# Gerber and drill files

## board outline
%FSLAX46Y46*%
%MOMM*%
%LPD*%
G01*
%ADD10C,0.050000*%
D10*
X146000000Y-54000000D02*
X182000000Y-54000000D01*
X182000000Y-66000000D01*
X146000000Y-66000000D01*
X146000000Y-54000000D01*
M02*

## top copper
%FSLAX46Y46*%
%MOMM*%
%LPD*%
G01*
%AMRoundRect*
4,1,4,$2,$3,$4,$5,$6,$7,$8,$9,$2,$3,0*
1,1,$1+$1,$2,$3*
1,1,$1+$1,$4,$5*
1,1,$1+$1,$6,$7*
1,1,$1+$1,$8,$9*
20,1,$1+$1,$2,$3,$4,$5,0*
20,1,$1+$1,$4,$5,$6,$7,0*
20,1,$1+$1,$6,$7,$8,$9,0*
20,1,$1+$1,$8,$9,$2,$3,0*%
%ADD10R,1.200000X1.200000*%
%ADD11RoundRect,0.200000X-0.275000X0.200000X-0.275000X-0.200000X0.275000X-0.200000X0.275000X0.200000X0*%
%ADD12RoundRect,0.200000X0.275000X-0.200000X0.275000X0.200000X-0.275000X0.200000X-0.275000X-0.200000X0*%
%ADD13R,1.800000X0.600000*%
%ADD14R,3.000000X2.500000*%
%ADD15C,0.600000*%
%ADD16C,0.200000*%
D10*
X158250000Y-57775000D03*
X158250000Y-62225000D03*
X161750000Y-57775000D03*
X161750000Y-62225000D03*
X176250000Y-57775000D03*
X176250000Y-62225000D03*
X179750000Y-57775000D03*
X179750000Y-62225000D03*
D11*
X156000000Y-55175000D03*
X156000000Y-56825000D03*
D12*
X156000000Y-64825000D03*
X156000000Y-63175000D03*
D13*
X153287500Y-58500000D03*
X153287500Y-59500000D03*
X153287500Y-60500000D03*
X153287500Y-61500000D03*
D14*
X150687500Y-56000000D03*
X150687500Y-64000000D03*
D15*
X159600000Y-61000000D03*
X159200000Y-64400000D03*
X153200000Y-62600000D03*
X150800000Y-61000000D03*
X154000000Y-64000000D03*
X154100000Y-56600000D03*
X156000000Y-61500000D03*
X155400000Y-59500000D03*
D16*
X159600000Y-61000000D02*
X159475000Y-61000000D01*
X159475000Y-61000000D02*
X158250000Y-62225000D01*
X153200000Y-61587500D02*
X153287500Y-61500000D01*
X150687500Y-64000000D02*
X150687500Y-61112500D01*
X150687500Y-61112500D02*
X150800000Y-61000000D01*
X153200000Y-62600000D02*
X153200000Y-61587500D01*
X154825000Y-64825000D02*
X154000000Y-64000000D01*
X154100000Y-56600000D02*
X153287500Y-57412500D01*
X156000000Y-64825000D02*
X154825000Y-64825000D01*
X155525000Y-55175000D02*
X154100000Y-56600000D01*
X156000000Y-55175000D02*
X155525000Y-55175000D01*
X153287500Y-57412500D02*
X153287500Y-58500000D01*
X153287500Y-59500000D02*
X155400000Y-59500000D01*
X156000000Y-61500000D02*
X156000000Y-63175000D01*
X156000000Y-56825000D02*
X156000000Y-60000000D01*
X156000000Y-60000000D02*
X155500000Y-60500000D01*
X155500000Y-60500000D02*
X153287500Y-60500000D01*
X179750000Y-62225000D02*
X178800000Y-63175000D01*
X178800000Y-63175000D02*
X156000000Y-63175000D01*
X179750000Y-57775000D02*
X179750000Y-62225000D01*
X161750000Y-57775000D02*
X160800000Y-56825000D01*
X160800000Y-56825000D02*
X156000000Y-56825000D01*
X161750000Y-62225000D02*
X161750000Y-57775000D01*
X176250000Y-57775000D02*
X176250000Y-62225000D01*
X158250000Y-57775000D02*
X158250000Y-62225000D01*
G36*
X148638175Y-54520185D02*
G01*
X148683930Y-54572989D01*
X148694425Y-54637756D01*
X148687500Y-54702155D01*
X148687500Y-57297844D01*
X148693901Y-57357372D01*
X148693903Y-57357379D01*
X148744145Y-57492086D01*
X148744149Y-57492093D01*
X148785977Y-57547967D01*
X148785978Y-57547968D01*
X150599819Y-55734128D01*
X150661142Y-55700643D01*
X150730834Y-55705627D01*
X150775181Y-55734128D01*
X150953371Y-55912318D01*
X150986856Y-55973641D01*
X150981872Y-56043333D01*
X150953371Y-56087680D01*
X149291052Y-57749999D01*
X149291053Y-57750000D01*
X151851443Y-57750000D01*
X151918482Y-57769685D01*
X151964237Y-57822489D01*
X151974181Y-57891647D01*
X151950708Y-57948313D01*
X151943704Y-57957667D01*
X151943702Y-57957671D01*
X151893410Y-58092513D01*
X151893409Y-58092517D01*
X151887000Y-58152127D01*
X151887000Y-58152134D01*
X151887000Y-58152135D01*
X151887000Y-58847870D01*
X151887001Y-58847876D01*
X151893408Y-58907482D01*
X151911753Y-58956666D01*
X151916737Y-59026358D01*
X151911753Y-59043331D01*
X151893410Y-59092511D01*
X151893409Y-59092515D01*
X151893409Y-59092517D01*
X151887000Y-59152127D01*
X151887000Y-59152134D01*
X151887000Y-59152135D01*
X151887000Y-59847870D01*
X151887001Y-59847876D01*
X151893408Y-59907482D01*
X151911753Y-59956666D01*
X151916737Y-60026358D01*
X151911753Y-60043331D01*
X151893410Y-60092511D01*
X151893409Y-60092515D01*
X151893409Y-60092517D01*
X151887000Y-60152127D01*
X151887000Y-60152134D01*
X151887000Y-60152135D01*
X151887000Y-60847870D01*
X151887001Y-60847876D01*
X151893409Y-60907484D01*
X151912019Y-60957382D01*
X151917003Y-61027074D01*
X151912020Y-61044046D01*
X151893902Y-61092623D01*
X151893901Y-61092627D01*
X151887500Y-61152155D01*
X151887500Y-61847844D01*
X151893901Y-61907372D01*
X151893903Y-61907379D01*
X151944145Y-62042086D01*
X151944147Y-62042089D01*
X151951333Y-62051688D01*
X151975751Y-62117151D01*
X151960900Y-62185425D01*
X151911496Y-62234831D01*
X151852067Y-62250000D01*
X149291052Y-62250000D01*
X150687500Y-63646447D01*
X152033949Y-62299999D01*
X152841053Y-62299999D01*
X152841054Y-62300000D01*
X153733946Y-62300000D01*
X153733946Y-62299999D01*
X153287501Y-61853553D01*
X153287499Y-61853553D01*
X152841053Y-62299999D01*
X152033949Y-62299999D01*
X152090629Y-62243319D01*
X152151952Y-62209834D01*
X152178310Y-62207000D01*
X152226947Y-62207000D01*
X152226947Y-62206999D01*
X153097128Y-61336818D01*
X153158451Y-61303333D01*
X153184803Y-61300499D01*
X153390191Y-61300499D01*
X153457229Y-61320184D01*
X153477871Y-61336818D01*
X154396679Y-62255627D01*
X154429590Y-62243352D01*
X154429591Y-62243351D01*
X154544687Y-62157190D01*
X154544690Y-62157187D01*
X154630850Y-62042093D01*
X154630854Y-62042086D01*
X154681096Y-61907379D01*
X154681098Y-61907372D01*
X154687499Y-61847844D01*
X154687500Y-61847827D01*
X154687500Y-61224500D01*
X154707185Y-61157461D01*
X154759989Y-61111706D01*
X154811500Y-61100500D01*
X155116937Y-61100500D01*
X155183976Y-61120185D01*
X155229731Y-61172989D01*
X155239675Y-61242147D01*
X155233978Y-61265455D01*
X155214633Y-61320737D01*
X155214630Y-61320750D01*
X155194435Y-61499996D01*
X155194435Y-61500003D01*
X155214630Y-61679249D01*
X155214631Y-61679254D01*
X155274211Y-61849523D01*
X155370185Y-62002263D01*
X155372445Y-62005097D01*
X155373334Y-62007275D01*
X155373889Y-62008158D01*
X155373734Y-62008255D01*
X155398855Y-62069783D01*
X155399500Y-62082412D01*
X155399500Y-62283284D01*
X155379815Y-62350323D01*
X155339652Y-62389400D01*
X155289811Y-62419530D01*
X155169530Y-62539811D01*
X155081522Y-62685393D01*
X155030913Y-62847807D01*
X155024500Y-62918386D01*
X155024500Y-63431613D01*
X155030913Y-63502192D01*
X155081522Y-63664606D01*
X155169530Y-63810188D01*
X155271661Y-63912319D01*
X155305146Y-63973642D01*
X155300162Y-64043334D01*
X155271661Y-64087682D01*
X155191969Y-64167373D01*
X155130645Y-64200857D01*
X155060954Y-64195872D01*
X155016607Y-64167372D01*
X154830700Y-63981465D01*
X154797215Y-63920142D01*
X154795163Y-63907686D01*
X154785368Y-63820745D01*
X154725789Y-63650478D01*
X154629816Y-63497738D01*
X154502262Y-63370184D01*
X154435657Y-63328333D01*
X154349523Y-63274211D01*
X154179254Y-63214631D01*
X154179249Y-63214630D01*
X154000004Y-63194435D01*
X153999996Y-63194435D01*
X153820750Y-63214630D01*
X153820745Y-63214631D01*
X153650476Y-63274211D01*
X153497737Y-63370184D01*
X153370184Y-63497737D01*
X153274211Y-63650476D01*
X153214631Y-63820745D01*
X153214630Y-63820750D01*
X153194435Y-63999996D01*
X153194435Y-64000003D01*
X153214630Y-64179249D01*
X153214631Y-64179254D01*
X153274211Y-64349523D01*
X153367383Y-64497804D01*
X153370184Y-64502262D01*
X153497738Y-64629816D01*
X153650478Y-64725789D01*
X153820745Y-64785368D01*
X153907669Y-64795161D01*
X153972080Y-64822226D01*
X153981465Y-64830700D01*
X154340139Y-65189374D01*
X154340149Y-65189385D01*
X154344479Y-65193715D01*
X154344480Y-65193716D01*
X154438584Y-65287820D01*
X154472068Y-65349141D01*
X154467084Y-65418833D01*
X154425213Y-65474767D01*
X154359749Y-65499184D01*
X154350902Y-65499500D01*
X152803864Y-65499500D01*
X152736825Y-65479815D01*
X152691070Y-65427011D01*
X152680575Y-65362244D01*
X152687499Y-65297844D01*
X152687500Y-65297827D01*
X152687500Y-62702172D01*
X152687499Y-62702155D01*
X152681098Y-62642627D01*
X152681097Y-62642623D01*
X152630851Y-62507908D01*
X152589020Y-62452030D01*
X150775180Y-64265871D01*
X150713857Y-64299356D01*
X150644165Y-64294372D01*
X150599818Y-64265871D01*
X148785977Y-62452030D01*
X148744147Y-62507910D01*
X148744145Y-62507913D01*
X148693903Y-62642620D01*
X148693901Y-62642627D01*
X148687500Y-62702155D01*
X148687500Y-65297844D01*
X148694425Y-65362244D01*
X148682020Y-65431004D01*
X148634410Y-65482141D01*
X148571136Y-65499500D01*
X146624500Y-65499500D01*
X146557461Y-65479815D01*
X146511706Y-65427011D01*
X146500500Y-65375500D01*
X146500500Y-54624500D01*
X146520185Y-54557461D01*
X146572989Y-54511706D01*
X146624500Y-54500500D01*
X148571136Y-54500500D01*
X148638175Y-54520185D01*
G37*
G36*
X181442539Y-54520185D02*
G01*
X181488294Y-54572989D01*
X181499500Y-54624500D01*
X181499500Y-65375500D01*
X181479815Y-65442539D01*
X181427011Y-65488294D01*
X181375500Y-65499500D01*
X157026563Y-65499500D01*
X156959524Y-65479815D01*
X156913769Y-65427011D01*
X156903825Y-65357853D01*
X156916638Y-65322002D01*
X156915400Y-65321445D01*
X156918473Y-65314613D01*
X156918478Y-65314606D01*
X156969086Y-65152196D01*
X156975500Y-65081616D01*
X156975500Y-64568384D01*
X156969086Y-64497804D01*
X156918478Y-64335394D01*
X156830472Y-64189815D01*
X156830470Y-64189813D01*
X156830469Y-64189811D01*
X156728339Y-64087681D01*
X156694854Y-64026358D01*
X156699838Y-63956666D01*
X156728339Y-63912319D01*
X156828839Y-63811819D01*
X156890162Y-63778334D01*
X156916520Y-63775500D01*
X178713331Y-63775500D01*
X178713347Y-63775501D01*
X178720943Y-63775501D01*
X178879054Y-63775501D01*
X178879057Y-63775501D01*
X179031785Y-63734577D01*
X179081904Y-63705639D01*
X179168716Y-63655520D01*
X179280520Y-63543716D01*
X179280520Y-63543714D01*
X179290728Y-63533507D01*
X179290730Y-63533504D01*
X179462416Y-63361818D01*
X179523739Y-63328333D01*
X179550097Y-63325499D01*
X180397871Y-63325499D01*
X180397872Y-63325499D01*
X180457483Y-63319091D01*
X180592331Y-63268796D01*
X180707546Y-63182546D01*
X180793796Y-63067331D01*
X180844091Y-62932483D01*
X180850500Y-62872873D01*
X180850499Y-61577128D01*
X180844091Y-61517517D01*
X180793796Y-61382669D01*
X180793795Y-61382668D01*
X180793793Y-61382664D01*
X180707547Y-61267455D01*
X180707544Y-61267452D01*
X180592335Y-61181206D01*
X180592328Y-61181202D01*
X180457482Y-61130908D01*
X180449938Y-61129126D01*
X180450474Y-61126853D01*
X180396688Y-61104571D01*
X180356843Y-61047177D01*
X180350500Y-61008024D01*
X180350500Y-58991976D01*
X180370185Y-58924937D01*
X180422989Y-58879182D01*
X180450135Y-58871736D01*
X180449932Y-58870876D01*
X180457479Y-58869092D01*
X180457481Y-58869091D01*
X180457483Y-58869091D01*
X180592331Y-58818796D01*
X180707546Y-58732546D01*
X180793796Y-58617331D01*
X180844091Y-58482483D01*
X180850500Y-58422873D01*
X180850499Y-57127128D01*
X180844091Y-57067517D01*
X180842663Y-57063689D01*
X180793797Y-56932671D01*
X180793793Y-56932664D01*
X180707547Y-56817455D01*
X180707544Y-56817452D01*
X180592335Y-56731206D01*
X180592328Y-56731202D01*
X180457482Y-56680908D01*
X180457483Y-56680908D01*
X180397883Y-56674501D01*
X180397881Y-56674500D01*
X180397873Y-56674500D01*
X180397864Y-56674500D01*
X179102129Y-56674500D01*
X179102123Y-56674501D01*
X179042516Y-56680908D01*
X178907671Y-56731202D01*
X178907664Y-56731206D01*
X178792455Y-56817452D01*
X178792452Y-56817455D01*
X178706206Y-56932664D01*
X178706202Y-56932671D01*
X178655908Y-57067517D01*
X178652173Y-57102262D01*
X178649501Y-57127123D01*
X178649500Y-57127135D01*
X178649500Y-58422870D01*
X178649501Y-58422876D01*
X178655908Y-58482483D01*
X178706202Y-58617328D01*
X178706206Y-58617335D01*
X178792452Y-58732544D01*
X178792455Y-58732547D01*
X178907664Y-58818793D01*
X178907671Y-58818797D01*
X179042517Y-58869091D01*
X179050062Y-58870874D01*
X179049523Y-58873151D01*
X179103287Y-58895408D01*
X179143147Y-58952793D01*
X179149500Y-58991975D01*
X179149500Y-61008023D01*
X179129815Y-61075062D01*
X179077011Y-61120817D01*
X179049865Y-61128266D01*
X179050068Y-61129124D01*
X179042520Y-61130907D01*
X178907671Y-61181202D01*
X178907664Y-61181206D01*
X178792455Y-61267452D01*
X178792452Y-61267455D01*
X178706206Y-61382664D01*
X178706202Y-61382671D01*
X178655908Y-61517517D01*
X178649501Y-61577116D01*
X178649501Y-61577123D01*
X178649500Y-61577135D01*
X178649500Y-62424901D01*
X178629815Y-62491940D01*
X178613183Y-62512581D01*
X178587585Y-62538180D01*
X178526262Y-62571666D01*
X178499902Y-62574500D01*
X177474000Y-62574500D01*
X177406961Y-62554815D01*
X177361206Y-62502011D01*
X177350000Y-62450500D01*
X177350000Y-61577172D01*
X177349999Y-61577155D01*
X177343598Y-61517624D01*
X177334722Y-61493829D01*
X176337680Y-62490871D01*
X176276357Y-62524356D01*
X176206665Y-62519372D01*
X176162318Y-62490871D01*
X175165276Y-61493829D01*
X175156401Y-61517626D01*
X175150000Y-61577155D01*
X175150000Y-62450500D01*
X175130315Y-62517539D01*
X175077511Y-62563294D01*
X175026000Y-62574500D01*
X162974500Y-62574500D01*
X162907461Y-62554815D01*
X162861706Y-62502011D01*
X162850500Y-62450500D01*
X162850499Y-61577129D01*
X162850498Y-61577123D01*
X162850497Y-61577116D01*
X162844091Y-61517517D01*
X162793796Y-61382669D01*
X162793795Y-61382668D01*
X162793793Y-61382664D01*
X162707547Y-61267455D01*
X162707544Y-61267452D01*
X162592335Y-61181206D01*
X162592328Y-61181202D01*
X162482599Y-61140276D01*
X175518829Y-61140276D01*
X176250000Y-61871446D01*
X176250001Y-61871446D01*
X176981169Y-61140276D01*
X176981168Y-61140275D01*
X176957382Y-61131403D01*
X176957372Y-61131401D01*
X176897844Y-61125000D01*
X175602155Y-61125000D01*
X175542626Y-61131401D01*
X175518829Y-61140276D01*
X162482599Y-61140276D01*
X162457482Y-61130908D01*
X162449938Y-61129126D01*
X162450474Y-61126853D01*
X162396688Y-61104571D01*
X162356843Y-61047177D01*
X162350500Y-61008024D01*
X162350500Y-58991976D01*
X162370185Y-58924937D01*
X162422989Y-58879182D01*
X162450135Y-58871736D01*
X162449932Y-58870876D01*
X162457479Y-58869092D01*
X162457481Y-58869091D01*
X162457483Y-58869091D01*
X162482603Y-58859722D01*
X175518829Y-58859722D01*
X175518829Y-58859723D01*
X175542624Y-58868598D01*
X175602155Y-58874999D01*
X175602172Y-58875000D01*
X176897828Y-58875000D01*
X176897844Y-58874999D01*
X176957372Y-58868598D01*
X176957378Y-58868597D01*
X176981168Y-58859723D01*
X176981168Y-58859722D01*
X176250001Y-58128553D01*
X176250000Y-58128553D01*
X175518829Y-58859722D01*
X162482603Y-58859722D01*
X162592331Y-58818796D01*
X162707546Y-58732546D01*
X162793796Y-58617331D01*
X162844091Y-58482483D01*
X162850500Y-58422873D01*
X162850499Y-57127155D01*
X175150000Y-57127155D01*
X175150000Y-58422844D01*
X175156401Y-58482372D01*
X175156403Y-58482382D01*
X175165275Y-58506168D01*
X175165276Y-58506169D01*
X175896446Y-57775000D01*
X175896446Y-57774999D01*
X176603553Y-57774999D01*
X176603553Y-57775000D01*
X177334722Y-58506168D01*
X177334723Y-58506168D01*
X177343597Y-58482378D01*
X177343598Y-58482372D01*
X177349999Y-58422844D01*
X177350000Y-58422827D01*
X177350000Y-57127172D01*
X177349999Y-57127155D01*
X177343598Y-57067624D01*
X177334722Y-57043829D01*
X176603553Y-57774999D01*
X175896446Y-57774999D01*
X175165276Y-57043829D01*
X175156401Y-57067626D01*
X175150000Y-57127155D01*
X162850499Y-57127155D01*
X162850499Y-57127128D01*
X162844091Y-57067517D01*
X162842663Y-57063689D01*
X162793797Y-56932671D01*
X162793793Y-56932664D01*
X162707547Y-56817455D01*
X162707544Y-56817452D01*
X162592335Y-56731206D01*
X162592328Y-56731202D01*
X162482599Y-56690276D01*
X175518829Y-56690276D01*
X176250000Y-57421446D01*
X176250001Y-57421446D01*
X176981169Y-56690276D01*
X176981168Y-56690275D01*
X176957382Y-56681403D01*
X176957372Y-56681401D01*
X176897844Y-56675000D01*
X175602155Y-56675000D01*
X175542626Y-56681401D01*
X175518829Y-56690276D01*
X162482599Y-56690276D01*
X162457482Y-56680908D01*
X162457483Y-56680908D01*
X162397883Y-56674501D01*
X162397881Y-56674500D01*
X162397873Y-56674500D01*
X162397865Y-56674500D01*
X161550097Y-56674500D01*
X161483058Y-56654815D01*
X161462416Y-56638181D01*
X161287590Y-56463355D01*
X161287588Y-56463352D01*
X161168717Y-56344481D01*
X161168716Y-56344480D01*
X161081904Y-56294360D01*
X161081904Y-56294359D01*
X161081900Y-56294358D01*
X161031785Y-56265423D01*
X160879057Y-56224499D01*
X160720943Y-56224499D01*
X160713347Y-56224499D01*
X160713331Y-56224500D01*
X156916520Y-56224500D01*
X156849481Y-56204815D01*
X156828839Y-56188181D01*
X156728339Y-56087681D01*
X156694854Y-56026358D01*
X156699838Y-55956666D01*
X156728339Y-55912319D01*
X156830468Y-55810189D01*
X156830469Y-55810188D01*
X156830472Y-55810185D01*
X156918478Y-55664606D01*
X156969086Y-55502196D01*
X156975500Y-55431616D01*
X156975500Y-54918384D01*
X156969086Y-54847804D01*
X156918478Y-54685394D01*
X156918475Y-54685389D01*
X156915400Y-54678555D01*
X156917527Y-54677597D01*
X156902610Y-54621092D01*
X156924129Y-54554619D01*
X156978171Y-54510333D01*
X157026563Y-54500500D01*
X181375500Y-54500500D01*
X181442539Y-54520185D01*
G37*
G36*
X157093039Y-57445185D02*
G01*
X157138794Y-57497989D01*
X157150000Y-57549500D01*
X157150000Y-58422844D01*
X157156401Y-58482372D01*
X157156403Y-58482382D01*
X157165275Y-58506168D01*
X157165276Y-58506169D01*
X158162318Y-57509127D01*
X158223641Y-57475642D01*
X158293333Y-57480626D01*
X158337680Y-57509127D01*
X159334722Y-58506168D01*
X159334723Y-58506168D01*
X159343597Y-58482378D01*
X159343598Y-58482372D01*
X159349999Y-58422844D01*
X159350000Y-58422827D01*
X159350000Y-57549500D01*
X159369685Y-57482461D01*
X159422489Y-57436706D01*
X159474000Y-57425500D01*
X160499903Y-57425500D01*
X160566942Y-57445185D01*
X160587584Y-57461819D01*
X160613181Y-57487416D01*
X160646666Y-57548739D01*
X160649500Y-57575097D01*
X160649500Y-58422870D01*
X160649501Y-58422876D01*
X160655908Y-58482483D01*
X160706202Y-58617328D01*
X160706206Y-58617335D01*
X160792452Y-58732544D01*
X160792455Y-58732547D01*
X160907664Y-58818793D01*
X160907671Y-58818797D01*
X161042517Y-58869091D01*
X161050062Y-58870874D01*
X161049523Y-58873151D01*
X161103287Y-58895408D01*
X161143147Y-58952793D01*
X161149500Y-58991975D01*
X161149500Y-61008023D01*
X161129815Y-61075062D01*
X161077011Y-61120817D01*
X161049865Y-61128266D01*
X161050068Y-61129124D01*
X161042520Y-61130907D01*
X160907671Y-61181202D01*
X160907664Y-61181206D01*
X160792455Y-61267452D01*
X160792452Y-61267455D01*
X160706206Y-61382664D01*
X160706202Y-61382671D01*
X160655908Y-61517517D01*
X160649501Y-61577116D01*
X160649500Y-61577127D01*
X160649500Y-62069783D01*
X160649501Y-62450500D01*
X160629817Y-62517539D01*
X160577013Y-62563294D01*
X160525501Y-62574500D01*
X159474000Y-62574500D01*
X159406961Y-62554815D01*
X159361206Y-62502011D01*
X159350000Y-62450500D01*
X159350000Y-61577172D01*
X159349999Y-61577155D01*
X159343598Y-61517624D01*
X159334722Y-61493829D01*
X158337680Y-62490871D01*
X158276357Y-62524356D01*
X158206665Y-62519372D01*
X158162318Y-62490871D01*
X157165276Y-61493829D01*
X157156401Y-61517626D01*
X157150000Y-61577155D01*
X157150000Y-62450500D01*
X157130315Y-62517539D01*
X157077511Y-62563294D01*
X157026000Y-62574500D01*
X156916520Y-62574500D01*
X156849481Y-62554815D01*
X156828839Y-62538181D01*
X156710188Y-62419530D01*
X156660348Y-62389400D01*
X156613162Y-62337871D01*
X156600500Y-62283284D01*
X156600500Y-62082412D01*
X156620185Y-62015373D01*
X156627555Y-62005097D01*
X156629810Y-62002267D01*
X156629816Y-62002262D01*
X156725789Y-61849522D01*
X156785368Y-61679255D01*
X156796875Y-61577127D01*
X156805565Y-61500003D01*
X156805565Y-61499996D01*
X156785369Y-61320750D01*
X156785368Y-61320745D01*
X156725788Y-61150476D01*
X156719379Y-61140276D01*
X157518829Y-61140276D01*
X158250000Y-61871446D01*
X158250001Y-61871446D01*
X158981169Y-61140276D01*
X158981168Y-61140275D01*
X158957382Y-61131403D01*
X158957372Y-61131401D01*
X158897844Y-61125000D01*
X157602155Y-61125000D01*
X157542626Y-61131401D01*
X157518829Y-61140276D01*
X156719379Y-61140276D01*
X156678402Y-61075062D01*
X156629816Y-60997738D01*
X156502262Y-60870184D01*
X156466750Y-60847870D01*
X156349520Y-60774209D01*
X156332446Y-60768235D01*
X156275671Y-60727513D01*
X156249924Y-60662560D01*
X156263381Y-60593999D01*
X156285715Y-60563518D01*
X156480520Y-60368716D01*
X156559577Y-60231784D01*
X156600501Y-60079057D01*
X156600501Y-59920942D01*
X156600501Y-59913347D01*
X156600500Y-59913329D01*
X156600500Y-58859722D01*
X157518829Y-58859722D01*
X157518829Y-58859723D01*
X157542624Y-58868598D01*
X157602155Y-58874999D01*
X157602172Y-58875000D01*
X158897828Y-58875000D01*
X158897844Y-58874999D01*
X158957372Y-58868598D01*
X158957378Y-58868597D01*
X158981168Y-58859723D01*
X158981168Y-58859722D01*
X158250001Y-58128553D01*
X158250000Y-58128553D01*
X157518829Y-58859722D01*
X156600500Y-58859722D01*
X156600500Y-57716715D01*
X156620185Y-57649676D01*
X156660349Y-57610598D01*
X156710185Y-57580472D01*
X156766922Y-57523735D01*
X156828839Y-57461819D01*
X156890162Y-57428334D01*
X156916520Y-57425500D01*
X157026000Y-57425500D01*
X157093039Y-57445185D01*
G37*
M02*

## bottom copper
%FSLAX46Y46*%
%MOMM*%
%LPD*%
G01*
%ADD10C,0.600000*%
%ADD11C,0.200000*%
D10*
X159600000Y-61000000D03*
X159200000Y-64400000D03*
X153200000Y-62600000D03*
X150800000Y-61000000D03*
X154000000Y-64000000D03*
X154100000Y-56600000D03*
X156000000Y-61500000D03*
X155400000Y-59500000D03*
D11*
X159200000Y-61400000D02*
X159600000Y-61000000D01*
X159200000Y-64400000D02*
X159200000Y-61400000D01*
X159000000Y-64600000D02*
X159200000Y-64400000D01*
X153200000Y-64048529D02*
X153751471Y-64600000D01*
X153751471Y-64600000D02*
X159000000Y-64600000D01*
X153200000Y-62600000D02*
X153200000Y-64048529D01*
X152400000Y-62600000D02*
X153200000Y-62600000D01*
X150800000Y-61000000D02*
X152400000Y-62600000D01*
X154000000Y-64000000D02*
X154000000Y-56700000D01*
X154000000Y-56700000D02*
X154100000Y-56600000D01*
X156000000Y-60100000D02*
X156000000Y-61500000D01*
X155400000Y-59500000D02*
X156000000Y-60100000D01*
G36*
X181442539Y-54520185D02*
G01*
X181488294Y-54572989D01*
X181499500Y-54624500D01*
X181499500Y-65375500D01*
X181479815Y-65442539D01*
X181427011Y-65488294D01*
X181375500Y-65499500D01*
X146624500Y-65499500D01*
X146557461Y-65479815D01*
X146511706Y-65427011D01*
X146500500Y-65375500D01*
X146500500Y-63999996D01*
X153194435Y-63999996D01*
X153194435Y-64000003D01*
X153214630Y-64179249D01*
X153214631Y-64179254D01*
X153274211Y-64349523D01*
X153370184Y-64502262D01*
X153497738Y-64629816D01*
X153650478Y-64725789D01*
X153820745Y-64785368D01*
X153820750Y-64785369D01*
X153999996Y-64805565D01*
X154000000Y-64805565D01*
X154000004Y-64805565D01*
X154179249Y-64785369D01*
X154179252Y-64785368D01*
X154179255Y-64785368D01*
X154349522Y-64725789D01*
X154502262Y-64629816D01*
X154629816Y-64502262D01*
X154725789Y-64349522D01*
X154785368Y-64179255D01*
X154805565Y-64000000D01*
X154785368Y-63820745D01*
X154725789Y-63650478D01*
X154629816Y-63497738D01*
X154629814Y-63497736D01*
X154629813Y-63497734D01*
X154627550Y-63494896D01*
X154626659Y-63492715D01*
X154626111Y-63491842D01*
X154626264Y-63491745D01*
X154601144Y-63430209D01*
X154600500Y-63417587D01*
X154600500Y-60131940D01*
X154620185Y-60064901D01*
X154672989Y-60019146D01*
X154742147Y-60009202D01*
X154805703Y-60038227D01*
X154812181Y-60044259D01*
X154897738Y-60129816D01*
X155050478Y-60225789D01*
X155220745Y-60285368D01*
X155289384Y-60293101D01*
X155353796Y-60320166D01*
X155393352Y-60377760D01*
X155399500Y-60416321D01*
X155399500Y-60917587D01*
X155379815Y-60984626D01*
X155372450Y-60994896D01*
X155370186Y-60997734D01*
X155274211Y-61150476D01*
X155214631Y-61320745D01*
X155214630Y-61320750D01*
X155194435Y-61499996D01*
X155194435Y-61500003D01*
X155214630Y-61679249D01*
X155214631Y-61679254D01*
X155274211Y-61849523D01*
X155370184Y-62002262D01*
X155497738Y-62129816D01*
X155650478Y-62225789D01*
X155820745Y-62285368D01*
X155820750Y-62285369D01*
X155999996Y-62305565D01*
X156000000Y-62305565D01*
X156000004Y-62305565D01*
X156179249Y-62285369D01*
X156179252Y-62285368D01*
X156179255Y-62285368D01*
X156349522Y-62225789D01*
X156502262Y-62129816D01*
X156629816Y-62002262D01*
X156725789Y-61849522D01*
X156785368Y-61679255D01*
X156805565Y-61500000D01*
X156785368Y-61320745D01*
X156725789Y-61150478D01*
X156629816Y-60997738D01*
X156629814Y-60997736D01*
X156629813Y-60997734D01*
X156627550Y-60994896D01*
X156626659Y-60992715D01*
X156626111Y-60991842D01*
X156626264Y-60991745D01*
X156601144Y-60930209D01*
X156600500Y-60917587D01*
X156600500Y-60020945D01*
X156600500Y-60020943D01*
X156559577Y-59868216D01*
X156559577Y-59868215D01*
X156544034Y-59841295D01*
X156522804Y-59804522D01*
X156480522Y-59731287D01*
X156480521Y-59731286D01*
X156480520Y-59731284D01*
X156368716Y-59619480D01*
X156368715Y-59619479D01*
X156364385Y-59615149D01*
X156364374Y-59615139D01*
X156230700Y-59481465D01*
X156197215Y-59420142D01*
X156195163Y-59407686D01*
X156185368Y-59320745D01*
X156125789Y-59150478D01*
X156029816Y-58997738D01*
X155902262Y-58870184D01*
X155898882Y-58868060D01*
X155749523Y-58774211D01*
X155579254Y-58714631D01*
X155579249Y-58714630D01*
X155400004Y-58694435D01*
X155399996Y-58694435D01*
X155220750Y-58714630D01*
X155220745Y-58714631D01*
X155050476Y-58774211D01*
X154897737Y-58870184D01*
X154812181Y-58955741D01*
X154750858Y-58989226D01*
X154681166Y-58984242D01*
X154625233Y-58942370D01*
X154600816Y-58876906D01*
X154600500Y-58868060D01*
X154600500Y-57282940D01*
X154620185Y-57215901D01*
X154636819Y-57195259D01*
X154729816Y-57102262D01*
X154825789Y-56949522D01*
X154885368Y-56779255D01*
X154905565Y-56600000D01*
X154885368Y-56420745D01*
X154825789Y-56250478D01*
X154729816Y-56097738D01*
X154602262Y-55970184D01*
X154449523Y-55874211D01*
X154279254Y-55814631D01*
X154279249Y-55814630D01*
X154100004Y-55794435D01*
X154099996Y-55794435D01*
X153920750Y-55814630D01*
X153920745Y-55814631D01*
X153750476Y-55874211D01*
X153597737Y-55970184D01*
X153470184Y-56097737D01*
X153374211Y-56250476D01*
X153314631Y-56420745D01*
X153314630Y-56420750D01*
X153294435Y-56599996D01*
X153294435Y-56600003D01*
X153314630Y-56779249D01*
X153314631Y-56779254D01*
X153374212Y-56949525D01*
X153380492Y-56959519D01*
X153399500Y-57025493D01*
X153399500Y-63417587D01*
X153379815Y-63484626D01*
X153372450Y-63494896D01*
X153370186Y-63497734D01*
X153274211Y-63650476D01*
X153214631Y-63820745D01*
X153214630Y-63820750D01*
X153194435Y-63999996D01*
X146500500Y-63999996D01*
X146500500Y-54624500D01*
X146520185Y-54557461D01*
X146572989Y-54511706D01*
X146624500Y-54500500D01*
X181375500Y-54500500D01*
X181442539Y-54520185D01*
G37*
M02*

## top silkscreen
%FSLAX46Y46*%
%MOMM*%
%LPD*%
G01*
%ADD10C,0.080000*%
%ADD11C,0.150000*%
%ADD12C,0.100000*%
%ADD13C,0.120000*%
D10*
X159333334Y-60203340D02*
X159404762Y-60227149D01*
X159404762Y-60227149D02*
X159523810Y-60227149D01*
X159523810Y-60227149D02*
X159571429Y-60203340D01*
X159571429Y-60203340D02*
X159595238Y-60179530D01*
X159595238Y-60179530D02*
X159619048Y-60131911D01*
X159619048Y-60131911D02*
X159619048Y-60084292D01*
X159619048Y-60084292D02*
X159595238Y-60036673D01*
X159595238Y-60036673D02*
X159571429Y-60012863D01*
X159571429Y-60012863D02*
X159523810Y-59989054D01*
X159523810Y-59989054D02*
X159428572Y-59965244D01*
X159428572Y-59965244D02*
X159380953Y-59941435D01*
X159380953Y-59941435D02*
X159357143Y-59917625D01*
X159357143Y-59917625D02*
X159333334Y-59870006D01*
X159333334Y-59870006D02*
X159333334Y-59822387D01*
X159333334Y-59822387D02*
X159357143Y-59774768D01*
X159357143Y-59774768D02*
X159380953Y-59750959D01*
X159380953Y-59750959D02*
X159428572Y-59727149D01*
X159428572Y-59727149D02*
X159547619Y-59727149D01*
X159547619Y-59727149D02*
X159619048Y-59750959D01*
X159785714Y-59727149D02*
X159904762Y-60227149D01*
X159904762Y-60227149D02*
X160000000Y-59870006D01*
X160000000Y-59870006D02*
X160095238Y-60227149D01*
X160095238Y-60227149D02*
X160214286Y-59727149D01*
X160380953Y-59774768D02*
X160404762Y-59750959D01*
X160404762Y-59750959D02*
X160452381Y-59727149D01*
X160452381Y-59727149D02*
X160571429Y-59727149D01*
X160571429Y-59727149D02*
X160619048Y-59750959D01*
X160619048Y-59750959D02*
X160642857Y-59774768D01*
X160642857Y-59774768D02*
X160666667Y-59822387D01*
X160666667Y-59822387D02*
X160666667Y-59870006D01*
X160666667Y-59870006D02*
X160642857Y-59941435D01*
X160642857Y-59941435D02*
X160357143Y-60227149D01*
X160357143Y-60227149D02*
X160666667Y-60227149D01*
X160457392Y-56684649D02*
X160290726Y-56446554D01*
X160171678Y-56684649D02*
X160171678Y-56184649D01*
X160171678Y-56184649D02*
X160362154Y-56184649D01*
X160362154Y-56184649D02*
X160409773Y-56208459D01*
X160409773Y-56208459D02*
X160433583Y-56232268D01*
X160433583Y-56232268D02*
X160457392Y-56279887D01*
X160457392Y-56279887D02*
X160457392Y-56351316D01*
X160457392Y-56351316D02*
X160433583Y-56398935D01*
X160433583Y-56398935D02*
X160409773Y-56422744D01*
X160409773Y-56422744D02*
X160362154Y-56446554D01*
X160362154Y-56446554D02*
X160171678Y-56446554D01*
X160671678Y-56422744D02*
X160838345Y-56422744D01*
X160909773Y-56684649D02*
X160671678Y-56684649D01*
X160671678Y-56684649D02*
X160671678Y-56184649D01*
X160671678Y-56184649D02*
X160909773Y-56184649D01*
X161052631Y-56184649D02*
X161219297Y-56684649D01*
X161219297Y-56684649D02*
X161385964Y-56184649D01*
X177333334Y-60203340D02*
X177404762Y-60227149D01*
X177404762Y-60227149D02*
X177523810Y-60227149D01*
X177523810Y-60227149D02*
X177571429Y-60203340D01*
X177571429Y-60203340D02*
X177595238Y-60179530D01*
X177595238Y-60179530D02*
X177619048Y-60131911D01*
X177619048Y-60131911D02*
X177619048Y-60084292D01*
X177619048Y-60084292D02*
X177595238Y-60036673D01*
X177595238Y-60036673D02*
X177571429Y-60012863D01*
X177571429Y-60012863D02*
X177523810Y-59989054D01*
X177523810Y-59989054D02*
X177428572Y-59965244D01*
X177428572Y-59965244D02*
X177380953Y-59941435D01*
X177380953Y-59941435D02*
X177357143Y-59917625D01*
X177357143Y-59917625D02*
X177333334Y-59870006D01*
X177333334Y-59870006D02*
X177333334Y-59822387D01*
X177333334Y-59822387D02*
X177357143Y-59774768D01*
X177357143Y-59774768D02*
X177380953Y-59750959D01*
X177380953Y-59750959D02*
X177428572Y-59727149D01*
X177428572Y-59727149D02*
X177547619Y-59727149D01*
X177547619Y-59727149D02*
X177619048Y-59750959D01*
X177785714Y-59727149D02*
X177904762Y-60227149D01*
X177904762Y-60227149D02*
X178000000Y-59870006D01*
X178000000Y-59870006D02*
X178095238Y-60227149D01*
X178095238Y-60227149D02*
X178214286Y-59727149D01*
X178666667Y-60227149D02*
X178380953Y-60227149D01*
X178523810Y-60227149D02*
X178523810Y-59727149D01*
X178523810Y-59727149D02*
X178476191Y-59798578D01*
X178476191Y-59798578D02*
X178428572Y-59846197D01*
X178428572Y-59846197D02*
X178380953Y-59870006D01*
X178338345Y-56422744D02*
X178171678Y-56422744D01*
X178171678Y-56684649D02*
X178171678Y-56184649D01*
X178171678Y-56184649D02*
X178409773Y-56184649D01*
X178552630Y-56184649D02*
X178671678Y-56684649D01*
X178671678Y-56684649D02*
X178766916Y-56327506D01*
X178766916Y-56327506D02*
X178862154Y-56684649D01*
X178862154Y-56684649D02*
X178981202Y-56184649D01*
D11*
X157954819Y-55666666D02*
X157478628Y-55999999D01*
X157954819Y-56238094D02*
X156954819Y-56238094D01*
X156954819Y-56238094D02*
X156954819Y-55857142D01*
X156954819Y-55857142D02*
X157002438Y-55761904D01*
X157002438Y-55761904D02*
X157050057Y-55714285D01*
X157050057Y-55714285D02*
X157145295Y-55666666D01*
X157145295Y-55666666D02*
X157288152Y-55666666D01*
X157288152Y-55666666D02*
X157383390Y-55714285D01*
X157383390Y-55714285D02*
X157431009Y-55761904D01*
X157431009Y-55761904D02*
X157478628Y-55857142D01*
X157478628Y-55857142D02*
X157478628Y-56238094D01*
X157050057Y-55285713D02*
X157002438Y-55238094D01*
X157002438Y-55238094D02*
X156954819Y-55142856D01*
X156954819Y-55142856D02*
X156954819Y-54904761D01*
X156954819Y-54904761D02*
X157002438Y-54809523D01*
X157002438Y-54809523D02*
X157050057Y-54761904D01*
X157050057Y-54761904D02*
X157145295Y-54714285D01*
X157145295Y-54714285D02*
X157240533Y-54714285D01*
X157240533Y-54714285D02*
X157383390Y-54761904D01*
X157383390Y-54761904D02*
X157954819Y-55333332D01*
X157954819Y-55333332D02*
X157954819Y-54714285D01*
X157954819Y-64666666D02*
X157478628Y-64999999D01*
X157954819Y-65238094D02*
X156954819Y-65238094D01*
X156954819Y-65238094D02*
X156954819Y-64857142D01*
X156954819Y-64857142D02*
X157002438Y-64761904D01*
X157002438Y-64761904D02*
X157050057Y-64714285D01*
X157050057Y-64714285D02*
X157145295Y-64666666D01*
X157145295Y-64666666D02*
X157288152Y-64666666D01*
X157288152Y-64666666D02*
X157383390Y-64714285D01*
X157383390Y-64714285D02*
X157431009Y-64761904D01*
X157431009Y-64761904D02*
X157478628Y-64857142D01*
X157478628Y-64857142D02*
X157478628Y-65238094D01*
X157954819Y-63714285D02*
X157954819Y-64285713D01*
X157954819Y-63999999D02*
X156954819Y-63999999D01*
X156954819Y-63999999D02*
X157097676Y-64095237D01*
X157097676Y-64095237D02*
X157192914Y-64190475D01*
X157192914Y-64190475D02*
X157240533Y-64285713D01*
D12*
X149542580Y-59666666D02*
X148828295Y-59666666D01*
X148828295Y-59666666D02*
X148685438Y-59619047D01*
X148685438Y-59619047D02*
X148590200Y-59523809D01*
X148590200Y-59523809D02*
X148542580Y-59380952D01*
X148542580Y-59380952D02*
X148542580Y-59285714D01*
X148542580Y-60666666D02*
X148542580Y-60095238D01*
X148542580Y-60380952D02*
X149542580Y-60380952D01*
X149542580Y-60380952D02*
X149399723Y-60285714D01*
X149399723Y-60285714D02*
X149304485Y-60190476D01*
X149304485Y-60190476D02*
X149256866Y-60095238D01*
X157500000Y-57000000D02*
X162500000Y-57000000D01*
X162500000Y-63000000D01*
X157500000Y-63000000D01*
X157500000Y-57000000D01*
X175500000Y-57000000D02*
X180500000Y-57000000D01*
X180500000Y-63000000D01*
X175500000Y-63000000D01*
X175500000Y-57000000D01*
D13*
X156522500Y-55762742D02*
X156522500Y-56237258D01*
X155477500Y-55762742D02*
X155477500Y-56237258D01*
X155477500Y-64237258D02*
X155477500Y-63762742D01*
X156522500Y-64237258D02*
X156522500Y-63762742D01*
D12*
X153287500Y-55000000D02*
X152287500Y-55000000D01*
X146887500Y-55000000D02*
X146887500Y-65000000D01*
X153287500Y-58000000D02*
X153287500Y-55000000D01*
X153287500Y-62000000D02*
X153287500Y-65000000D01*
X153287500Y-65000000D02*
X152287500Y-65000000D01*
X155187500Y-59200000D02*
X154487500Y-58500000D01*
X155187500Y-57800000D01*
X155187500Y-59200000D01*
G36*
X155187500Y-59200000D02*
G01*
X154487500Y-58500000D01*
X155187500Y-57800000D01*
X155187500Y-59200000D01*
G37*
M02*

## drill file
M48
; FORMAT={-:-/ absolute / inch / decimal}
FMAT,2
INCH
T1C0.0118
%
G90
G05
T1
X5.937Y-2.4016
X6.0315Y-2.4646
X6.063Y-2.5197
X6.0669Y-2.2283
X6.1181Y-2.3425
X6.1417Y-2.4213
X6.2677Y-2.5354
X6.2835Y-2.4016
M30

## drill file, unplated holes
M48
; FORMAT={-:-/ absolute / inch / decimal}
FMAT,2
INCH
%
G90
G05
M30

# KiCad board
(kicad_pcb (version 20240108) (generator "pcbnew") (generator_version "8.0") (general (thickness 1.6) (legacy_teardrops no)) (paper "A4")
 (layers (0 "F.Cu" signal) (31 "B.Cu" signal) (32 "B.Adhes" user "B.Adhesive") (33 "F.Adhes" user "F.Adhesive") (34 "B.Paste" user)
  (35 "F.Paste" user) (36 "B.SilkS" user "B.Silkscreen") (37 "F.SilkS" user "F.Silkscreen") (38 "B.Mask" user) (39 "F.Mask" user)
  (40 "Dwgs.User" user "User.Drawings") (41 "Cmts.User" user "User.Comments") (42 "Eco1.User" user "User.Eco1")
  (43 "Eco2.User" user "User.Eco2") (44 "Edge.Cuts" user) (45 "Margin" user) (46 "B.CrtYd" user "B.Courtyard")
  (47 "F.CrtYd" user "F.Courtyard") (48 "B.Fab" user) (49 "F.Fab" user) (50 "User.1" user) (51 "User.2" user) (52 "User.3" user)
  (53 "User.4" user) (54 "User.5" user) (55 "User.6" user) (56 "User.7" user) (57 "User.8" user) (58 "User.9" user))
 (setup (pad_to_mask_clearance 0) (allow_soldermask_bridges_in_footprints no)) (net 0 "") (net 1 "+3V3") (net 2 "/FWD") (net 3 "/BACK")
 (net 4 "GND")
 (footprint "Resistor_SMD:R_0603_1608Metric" (layer "F.Cu") (at 156 64 90)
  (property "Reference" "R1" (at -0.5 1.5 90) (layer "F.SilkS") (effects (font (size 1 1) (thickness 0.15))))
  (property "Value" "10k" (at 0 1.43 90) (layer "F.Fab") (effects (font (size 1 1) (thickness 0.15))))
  (fp_line (start -0.237258 -0.5225) (end 0.237258 -0.5225) (stroke (width 0.12) (type solid)) (layer "F.SilkS"))
  (fp_line (start -0.237258 0.5225) (end 0.237258 0.5225) (stroke (width 0.12) (type solid)) (layer "F.SilkS"))
  (pad "1" smd roundrect (at -0.825 0 90) (size 0.8 0.95) (layers "F.Cu" "F.Paste" "F.Mask") (roundrect_rratio 0.25) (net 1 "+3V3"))
  (pad "2" smd roundrect (at 0.825 0 90) (size 0.8 0.95) (layers "F.Cu" "F.Paste" "F.Mask") (roundrect_rratio 0.25) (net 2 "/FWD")))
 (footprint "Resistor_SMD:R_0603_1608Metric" (layer "F.Cu") (at 156 56 -90)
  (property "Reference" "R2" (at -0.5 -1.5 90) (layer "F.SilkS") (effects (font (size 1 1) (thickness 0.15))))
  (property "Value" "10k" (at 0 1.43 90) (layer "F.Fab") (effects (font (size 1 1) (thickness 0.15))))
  (fp_line (start -0.237258 0.5225) (end 0.237258 0.5225) (stroke (width 0.12) (type solid)) (layer "F.SilkS"))
  (fp_line (start -0.237258 -0.5225) (end 0.237258 -0.5225) (stroke (width 0.12) (type solid)) (layer "F.SilkS"))
  (pad "1" smd roundrect (at -0.825 0 270) (size 0.8 0.95) (layers "F.Cu" "F.Paste" "F.Mask") (roundrect_rratio 0.25) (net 1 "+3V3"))
  (pad "2" smd roundrect (at 0.825 0 270) (size 0.8 0.95) (layers "F.Cu" "F.Paste" "F.Mask") (roundrect_rratio 0.25) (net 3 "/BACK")))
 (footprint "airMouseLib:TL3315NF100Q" (layer "F.Cu") (at 178 60)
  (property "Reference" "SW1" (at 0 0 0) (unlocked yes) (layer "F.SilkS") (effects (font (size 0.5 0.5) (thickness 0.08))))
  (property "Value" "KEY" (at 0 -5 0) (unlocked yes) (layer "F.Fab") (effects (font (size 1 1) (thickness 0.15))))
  (fp_rect (start -2.5 -3) (end 2.5 3) (stroke (width 0.1) (type default)) (fill none) (layer "F.SilkS"))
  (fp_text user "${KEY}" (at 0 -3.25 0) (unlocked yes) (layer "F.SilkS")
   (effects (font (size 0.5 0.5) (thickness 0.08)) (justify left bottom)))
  (pad "1" smd rect (at -1.75 -2.225) (size 1.2 1.2) (layers "F.Cu" "F.Paste" "F.Mask") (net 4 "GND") (thermal_bridge_angle 45))
  (pad "1" smd rect (at -1.75 2.225 180) (size 1.2 1.2) (layers "F.Cu" "F.Paste" "F.Mask") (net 4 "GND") (thermal_bridge_angle 45))
  (pad "2" smd rect (at 1.75 -2.225) (size 1.2 1.2) (layers "F.Cu" "F.Paste" "F.Mask") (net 2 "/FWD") (thermal_bridge_angle 45))
  (pad "2" smd rect (at 1.75 2.225 180) (size 1.2 1.2) (layers "F.Cu" "F.Paste" "F.Mask") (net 2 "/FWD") (thermal_bridge_angle 45)))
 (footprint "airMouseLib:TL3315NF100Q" (layer "F.Cu") (at 160 60)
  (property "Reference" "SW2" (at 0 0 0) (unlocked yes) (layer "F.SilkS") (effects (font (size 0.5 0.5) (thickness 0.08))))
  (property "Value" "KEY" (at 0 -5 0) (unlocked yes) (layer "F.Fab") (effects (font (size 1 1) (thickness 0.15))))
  (fp_rect (start -2.5 -3) (end 2.5 3) (stroke (width 0.1) (type default)) (fill none) (layer "F.SilkS"))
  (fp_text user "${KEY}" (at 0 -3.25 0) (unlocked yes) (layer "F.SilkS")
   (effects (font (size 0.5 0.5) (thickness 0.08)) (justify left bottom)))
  (pad "1" smd rect (at -1.75 -2.225) (size 1.2 1.2) (layers "F.Cu" "F.Paste" "F.Mask") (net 4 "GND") (thermal_bridge_angle 45))
  (pad "1" smd rect (at -1.75 2.225 180) (size 1.2 1.2) (layers "F.Cu" "F.Paste" "F.Mask") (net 4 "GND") (thermal_bridge_angle 45))
  (pad "2" smd rect (at 1.75 -2.225) (size 1.2 1.2) (layers "F.Cu" "F.Paste" "F.Mask") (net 3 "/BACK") (thermal_bridge_angle 45))
  (pad "2" smd rect (at 1.75 2.225 180) (size 1.2 1.2) (layers "F.Cu" "F.Paste" "F.Mask") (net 3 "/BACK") (thermal_bridge_angle 45)))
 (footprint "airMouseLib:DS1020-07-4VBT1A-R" (layer "F.Cu") (at 153.2875 60 -90)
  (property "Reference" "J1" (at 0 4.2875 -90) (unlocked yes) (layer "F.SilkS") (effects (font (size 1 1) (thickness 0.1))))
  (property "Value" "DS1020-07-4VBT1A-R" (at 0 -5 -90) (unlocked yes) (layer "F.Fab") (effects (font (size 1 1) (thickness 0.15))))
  (fp_line (start -5 6.4) (end 5 6.4) (stroke (width 0.1) (type default)) (layer "F.SilkS"))
  (fp_line (start -5 0) (end -5 1) (stroke (width 0.1) (type default)) (layer "F.SilkS"))
  (fp_line (start -2 0) (end -5 0) (stroke (width 0.1) (type default)) (layer "F.SilkS"))
  (fp_line (start 2 0) (end 5 0) (stroke (width 0.1) (type default)) (layer "F.SilkS"))
  (fp_line (start 5 0) (end 5 1) (stroke (width 0.1) (type default)) (layer "F.SilkS"))
  (fp_poly (pts (xy -1.5 -1.2) (xy -2.2 -1.9) (xy -0.8 -1.9)) (stroke (width 0.1) (type solid)) (fill solid) (layer "F.SilkS"))
  (pad "1" smd rect (at -1.5 0 270) (size 0.6 1.8) (layers "F.Cu" "F.Paste" "F.Mask") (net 1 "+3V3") (thermal_bridge_angle 45))
  (pad "2" smd rect (at -0.5 0 270) (size 0.6 1.8) (layers "F.Cu" "F.Paste" "F.Mask") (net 2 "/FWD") (thermal_bridge_angle 45))
  (pad "3" smd rect (at 0.5 0 270) (size 0.6 1.8) (layers "F.Cu" "F.Paste" "F.Mask") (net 3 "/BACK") (thermal_bridge_angle 45))
  (pad "4" smd rect (at 1.5 0 270) (size 0.6 1.8) (layers "F.Cu" "F.Paste" "F.Mask") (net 4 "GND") (thermal_bridge_angle 45))
  (pad "MP" smd rect (at -4 2.6 270) (size 2.5 3) (layers "F.Cu" "F.Paste" "F.Mask") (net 4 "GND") (thermal_bridge_angle 45))
  (pad "MP" smd rect (at 4 2.6 270) (size 2.5 3) (layers "F.Cu" "F.Paste" "F.Mask") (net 4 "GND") (thermal_bridge_angle 45)))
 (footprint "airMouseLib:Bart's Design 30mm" (layer "B.Cu") (at 163.8 60.4 180)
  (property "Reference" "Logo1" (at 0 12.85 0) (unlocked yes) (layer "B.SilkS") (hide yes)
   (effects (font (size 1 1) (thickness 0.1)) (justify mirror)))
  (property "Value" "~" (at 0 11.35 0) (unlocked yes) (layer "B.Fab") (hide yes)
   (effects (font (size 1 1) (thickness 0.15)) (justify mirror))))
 (gr_rect (start 146 54) (end 182 66) (stroke (width 0.05) (type default)) (fill none) (layer "Edge.Cuts"))
 (segment (start 159.475 61) (end 158.25 62.225) (width 0.2) (layer "F.Cu") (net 4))
 (segment (start 153.2 61.5875) (end 153.2875 61.5) (width 0.2) (layer "F.Cu") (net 4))
 (segment (start 159.6 61) (end 159.475 61) (width 0.2) (layer "F.Cu") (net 4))
 (segment (start 153.2 62.6) (end 153.2 61.5875) (width 0.2) (layer "F.Cu") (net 4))
 (segment (start 158.25 57.775) (end 158.25 62.225) (width 0.2) (layer "F.Cu") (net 4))
 (segment (start 150.6875 64) (end 150.6875 61.1125) (width 0.2) (layer "F.Cu") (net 4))
 (segment (start 176.25 57.775) (end 176.25 62.225) (width 0.2) (layer "F.Cu") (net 4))
 (segment (start 150.6875 61.1125) (end 150.8 61) (width 0.2) (layer "F.Cu") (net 4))
 (via (at 150.8 61) (size 0.6) (drill 0.3) (layers "F.Cu" "B.Cu") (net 4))
 (via (at 153.2 62.6) (size 0.6) (drill 0.3) (layers "F.Cu" "B.Cu") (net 4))
 (via (at 159.6 61) (size 0.6) (drill 0.3) (layers "F.Cu" "B.Cu") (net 4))
 (via (at 159.2 64.4) (size 0.6) (drill 0.3) (layers "F.Cu" "B.Cu") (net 4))
 (segment (start 153.751471 64.6) (end 159 64.6) (width 0.2) (layer "B.Cu") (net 4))
 (segment (start 159 64.6) (end 159.2 64.4) (width 0.2) (layer "B.Cu") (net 4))
 (segment (start 159.2 64.4) (end 159.2 61.4) (width 0.2) (layer "B.Cu") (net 4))
 (segment (start 152.4 62.6) (end 153.2 62.6) (width 0.2) (layer "B.Cu") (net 4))
 (segment (start 153.2 64.048529) (end 153.751471 64.6) (width 0.2) (layer "B.Cu") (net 4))
 (segment (start 159.2 61.4) (end 159.6 61) (width 0.2) (layer "B.Cu") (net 4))
 (segment (start 150.8 61) (end 152.4 62.6) (width 0.2) (layer "B.Cu") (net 4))
 (segment (start 153.2 62.6) (end 153.2 64.048529) (width 0.2) (layer "B.Cu") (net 4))
 (segment (start 154.825 64.825) (end 154 64) (width 0.2) (layer "F.Cu") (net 1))
 (segment (start 156 64.825) (end 154.825 64.825) (width 0.2) (layer "F.Cu") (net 1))
 (segment (start 153.2875 57.4125) (end 153.2875 58.5) (width 0.2) (layer "F.Cu") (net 1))
 (segment (start 155.525 55.175) (end 154.1 56.6) (width 0.2) (layer "F.Cu") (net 1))
 (segment (start 156 55.175) (end 155.525 55.175) (width 0.2) (layer "F.Cu") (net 1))
 (segment (start 154.1 56.6) (end 153.2875 57.4125) (width 0.2) (layer "F.Cu") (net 1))
 (via (at 154.1 56.6) (size 0.6) (drill 0.3) (layers "F.Cu" "B.Cu") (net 1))
 (via (at 154 64) (size 0.6) (drill 0.3) (layers "F.Cu" "B.Cu") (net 1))
 (segment (start 154 64) (end 154 56.7) (width 0.2) (layer "B.Cu") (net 1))
 (segment (start 154 56.7) (end 154.1 56.6) (width 0.2) (layer "B.Cu") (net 1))
 (segment (start 156 61.5) (end 156 63.175) (width 0.2) (layer "F.Cu") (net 2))
 (segment (start 179.75 57.775) (end 179.75 62.225) (width 0.2) (layer "F.Cu") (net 2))
 (segment (start 179.75 62.225) (end 178.8 63.175) (width 0.2) (layer "F.Cu") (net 2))
 (segment (start 178.8 63.175) (end 156 63.175) (width 0.2) (layer "F.Cu") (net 2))
 (segment (start 153.2875 59.5) (end 155.4 59.5) (width 0.2) (layer "F.Cu") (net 2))
 (via (at 155.4 59.5) (size 0.6) (drill 0.3) (layers "F.Cu" "B.Cu") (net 2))
 (via (at 156 61.5) (size 0.6) (drill 0.3) (layers "F.Cu" "B.Cu") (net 2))
 (segment (start 155.4 59.5) (end 156 60.1) (width 0.2) (layer "B.Cu") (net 2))
 (segment (start 156 60.1) (end 156 61.5) (width 0.2) (layer "B.Cu") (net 2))
 (segment (start 155.5 60.5) (end 153.2875 60.5) (width 0.2) (layer "F.Cu") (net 3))
 (segment (start 160.8 56.825) (end 156 56.825) (width 0.2) (layer "F.Cu") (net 3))
 (segment (start 161.75 57.775) (end 160.8 56.825) (width 0.2) (layer "F.Cu") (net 3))
 (segment (start 156 60) (end 155.5 60.5) (width 0.2) (layer "F.Cu") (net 3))
 (segment (start 156 56.825) (end 156 60) (width 0.2) (layer "F.Cu") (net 3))
 (segment (start 161.75 62.225) (end 161.75 57.775) (width 0.2) (layer "F.Cu") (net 3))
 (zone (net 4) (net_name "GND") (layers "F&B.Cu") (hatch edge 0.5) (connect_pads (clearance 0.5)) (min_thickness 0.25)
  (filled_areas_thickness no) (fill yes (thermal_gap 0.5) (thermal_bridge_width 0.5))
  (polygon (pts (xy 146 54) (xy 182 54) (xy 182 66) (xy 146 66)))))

